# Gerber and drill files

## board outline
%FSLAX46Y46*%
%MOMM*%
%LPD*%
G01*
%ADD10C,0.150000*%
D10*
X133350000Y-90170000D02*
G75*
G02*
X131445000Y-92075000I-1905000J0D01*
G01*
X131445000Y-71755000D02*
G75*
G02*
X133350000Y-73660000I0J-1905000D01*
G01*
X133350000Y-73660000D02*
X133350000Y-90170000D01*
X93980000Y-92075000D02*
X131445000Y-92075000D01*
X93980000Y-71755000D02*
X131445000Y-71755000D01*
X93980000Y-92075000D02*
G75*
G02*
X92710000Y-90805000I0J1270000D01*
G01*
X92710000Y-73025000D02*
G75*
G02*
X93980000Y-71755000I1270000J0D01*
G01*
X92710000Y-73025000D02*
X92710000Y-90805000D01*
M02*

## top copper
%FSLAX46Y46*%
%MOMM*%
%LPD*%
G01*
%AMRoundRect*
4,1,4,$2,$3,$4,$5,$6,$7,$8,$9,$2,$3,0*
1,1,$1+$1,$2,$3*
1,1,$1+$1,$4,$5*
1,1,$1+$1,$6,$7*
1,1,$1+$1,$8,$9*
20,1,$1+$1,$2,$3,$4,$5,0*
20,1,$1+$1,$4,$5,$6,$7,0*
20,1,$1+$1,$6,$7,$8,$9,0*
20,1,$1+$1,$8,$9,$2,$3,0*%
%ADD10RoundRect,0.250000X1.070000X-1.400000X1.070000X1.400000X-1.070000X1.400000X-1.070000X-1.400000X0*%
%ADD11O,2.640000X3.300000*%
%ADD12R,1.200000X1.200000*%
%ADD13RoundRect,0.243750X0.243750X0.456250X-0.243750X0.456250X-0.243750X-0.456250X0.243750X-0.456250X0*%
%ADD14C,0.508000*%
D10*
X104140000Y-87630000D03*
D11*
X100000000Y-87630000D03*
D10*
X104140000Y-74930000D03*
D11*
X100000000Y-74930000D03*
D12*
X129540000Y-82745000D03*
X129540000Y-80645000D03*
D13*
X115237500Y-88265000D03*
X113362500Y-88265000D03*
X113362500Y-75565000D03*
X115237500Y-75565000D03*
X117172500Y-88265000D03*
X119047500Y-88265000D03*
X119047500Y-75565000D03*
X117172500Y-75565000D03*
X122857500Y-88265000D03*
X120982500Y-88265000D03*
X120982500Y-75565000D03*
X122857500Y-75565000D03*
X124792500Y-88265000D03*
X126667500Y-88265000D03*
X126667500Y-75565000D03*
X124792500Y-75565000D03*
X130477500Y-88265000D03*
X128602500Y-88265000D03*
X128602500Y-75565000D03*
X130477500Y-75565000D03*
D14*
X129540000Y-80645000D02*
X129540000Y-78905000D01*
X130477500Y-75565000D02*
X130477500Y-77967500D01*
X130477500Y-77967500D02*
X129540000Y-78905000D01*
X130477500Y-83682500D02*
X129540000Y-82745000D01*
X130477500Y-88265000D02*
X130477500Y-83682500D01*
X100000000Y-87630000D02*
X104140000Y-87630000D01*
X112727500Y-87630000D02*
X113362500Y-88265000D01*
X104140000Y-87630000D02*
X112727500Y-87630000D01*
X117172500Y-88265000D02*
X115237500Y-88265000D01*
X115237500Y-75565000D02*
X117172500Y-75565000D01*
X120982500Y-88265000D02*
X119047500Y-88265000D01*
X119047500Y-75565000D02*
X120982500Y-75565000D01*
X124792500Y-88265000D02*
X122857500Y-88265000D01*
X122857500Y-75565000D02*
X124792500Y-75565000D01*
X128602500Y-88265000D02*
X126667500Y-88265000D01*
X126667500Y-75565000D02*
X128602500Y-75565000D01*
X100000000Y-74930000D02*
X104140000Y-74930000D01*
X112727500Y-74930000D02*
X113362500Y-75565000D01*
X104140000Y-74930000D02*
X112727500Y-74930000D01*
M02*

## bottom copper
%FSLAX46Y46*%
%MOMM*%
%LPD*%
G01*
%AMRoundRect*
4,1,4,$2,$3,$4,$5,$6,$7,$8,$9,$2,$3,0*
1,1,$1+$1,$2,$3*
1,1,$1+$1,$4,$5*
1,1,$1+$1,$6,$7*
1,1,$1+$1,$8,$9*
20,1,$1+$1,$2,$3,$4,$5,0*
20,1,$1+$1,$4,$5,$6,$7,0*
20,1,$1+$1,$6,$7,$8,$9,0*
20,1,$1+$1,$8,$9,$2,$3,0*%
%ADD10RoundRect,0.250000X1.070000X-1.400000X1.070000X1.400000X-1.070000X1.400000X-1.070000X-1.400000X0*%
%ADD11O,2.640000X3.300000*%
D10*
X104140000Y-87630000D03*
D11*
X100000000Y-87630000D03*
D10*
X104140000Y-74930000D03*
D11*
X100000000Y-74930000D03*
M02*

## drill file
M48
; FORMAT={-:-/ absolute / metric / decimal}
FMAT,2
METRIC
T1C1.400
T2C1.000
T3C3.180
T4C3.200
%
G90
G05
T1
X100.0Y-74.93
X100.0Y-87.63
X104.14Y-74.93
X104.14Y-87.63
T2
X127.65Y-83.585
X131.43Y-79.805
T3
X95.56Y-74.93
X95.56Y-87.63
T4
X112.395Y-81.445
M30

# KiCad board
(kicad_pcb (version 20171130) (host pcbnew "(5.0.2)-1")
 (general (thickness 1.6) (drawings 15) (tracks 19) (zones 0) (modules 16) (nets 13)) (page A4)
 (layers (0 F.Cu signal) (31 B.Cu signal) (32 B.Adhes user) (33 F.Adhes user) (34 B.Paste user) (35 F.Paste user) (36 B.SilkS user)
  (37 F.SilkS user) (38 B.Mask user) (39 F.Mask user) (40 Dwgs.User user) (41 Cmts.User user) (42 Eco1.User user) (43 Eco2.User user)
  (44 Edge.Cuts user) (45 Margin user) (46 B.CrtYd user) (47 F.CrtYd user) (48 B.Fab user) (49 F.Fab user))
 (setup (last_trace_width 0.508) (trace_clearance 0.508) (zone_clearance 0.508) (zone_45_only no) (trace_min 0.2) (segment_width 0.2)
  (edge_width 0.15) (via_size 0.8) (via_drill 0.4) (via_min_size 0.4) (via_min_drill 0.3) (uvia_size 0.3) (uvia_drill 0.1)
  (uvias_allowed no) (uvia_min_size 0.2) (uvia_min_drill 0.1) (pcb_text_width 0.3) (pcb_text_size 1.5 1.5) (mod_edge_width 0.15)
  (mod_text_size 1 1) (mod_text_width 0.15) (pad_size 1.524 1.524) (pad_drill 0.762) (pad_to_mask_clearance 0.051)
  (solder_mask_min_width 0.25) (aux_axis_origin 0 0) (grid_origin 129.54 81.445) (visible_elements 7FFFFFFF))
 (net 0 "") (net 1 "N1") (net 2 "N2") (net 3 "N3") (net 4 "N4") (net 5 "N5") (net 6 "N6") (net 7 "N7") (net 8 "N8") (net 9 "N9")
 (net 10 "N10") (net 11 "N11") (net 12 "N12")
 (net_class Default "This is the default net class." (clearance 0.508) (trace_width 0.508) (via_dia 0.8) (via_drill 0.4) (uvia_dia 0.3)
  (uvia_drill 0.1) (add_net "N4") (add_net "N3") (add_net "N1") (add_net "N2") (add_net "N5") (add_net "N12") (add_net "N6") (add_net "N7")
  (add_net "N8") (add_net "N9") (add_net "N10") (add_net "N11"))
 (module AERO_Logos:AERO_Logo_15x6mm (layer F.Cu) (at 101.6 81.445)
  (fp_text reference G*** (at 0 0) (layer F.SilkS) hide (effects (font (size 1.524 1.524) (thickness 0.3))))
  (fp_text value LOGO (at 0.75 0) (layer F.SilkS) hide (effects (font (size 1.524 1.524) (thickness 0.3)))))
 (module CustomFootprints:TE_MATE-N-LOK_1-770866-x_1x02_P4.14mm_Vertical (layer B.Cu) (at 104.14 87.63 90)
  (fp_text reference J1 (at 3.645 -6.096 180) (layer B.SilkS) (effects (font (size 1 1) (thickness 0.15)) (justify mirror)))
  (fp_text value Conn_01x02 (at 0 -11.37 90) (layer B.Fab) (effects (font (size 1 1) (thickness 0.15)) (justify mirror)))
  (pad 1 thru_hole roundrect (at 0 0 90) (size 3.3 2.64) (drill 1.4) (layers *.Cu *.Mask) (roundrect_rratio 0.094697) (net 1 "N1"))
  (pad 2 thru_hole oval (at 0 -4.14 90) (size 3.3 2.64) (drill 1.4) (layers *.Cu *.Mask) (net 1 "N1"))
  (pad "" np_thru_hole circle (at 0 -8.58 90) (size 3.18 3.18) (drill 3.18) (layers *.Cu *.Mask)))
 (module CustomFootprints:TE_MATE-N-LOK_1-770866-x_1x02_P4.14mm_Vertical (layer B.Cu) (at 104.14 74.93 90)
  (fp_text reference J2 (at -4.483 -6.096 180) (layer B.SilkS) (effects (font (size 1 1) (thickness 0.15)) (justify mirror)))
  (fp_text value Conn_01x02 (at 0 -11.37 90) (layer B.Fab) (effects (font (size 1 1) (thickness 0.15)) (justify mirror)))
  (pad 1 thru_hole roundrect (at 0 0 90) (size 3.3 2.64) (drill 1.4) (layers *.Cu *.Mask) (roundrect_rratio 0.094697) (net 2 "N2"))
  (pad 2 thru_hole oval (at 0 -4.14 90) (size 3.3 2.64) (drill 1.4) (layers *.Cu *.Mask) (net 2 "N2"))
  (pad "" np_thru_hole circle (at 0 -8.58 90) (size 3.18 3.18) (drill 3.18) (layers *.Cu *.Mask)))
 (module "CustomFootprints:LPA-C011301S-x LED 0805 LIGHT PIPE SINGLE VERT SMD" (layer F.Cu) (at 129.54 81.695 270)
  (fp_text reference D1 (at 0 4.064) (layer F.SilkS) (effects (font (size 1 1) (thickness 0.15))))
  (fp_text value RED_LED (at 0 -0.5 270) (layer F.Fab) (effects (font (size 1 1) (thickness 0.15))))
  (pad "" np_thru_hole circle (at 1.89 1.89 270) (size 1 1) (drill 1) (layers *.Cu *.Mask))
  (pad "" np_thru_hole circle (at -1.89 -1.89 270) (size 1 1) (drill 1) (layers *.Cu *.Mask))
  (pad 2 smd rect (at 1.05 0 270) (size 1.2 1.2) (layers F.Cu F.Paste F.Mask) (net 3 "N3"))
  (pad 1 smd rect (at -1.05 0 270) (size 1.2 1.2) (layers F.Cu F.Paste F.Mask) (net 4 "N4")))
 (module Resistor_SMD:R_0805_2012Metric (layer F.Cu) (at 114.3 88.265 180)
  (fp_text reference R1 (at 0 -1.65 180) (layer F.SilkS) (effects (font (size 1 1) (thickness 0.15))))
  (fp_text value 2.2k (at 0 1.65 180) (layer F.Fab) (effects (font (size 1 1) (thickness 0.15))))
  (pad 1 smd roundrect (at -0.9375 0 180) (size 0.975 1.4) (layers F.Cu F.Paste F.Mask) (roundrect_rratio 0.25) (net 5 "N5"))
  (pad 2 smd roundrect (at 0.9375 0 180) (size 0.975 1.4) (layers F.Cu F.Paste F.Mask) (roundrect_rratio 0.25) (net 1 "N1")))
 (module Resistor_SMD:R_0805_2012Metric (layer F.Cu) (at 114.3 75.565 180)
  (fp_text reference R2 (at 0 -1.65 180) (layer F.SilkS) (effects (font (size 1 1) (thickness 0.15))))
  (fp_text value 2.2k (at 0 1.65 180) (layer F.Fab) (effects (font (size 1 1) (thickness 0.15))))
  (pad 2 smd roundrect (at 0.9375 0 180) (size 0.975 1.4) (layers F.Cu F.Paste F.Mask) (roundrect_rratio 0.25) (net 2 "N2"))
  (pad 1 smd roundrect (at -0.9375 0 180) (size 0.975 1.4) (layers F.Cu F.Paste F.Mask) (roundrect_rratio 0.25) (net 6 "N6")))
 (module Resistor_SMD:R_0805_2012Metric (layer F.Cu) (at 118.11 88.265 180)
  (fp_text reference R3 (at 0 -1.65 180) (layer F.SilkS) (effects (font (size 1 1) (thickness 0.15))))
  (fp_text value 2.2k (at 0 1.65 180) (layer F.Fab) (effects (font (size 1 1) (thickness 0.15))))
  (pad 2 smd roundrect (at 0.9375 0 180) (size 0.975 1.4) (layers F.Cu F.Paste F.Mask) (roundrect_rratio 0.25) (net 5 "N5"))
  (pad 1 smd roundrect (at -0.9375 0 180) (size 0.975 1.4) (layers F.Cu F.Paste F.Mask) (roundrect_rratio 0.25) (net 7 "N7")))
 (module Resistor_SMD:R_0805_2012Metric (layer F.Cu) (at 118.11 75.565 180)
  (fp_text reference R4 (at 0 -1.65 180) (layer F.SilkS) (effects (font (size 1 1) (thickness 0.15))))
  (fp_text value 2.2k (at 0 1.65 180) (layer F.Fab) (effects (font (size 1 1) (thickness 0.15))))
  (pad 1 smd roundrect (at -0.9375 0 180) (size 0.975 1.4) (layers F.Cu F.Paste F.Mask) (roundrect_rratio 0.25) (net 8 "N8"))
  (pad 2 smd roundrect (at 0.9375 0 180) (size 0.975 1.4) (layers F.Cu F.Paste F.Mask) (roundrect_rratio 0.25) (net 6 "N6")))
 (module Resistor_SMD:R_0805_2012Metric (layer F.Cu) (at 121.92 88.265 180)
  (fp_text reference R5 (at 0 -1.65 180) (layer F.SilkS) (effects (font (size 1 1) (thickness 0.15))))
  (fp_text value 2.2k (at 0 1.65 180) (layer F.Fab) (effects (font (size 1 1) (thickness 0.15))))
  (pad 1 smd roundrect (at -0.9375 0 180) (size 0.975 1.4) (layers F.Cu F.Paste F.Mask) (roundrect_rratio 0.25) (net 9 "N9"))
  (pad 2 smd roundrect (at 0.9375 0 180) (size 0.975 1.4) (layers F.Cu F.Paste F.Mask) (roundrect_rratio 0.25) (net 7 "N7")))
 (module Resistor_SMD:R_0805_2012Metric (layer F.Cu) (at 121.92 75.565 180)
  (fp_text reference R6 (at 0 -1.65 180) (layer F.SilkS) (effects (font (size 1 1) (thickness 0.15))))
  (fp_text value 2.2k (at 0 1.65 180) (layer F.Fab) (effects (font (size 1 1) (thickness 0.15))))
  (pad 2 smd roundrect (at 0.9375 0 180) (size 0.975 1.4) (layers F.Cu F.Paste F.Mask) (roundrect_rratio 0.25) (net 8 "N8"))
  (pad 1 smd roundrect (at -0.9375 0 180) (size 0.975 1.4) (layers F.Cu F.Paste F.Mask) (roundrect_rratio 0.25) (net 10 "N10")))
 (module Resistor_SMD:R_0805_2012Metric (layer F.Cu) (at 125.73 88.265 180)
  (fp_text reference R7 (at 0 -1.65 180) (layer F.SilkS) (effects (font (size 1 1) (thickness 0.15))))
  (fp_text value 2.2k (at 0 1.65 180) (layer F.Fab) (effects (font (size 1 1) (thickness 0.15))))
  (pad 2 smd roundrect (at 0.9375 0 180) (size 0.975 1.4) (layers F.Cu F.Paste F.Mask) (roundrect_rratio 0.25) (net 9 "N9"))
  (pad 1 smd roundrect (at -0.9375 0 180) (size 0.975 1.4) (layers F.Cu F.Paste F.Mask) (roundrect_rratio 0.25) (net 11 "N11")))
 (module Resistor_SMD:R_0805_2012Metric (layer F.Cu) (at 125.73 75.565 180)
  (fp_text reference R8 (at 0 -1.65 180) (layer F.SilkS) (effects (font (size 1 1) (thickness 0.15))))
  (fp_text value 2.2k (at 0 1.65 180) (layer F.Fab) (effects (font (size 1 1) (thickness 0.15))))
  (pad 1 smd roundrect (at -0.9375 0 180) (size 0.975 1.4) (layers F.Cu F.Paste F.Mask) (roundrect_rratio 0.25) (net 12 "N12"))
  (pad 2 smd roundrect (at 0.9375 0 180) (size 0.975 1.4) (layers F.Cu F.Paste F.Mask) (roundrect_rratio 0.25) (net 10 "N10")))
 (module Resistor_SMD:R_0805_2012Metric (layer F.Cu) (at 129.54 88.265 180)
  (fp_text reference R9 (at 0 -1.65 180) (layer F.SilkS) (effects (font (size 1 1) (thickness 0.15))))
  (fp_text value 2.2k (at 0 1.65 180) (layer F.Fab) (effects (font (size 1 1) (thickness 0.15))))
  (pad 1 smd roundrect (at -0.9375 0 180) (size 0.975 1.4) (layers F.Cu F.Paste F.Mask) (roundrect_rratio 0.25) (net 3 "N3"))
  (pad 2 smd roundrect (at 0.9375 0 180) (size 0.975 1.4) (layers F.Cu F.Paste F.Mask) (roundrect_rratio 0.25) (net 11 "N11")))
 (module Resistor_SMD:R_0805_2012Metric (layer F.Cu) (at 129.54 75.565 180)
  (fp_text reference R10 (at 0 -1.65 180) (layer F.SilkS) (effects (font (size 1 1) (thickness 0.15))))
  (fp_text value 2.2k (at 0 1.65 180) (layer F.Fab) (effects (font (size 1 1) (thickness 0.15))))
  (pad 2 smd roundrect (at 0.9375 0 180) (size 0.975 1.4) (layers F.Cu F.Paste F.Mask) (roundrect_rratio 0.25) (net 12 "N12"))
  (pad 1 smd roundrect (at -0.9375 0 180) (size 0.975 1.4) (layers F.Cu F.Paste F.Mask) (roundrect_rratio 0.25) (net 4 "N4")))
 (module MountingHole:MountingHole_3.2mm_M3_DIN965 (layer F.Cu) (at 112.395 81.445)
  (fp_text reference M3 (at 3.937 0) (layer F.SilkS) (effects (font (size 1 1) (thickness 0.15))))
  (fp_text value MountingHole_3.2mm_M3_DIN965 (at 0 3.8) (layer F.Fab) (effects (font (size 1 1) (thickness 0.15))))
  (pad 1 np_thru_hole circle (at 0 0) (size 3.2 3.2) (drill 3.2) (layers *.Cu *.Mask)))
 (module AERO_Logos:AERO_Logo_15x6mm (layer B.Cu) (at 122.936 77.381 180)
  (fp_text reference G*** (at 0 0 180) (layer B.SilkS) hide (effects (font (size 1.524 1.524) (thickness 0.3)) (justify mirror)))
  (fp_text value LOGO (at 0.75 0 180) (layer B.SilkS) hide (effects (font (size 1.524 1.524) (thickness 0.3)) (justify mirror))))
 (gr_arc (start 131.445 90.17) (end 131.445 92.075) (angle -90) (layer Edge.Cuts) (width 0.15))
 (gr_arc (start 131.445 73.66) (end 133.35 73.66) (angle -90) (layer Edge.Cuts) (width 0.15))
 (gr_line (start 133.35 73.66) (end 133.35 90.17) (layer Edge.Cuts) (width 0.15))
 (gr_line (start 93.98 92.075) (end 131.445 92.075) (layer Edge.Cuts) (width 0.15))
 (gr_line (start 93.98 71.755) (end 131.445 71.755) (layer Edge.Cuts) (width 0.15))
 (gr_arc (start 93.98 90.805) (end 92.71 90.805) (angle -90) (layer Edge.Cuts) (width 0.15))
 (gr_arc (start 93.98 73.025) (end 93.98 71.755) (angle -90) (layer Edge.Cuts) (width 0.15))
 (gr_line (start 92.71 73.025) (end 92.71 90.805) (layer Edge.Cuts) (width 0.15))
 (segment (start 129.54 80.645) (end 129.54 78.905) (width 0.508) (layer F.Cu) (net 4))
 (segment (start 130.4775 75.565) (end 130.4775 77.9675) (width 0.508) (layer F.Cu) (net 4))
 (segment (start 130.4775 77.9675) (end 129.54 78.905) (width 0.508) (layer F.Cu) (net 4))
 (segment (start 130.4775 83.6825) (end 129.54 82.745) (width 0.508) (layer F.Cu) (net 3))
 (segment (start 130.4775 88.265) (end 130.4775 83.6825) (width 0.508) (layer F.Cu) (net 3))
 (segment (start 100 87.63) (end 104.14 87.63) (width 0.508) (layer F.Cu) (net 1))
 (segment (start 112.7275 87.63) (end 113.3625 88.265) (width 0.508) (layer F.Cu) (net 1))
 (segment (start 104.14 87.63) (end 112.7275 87.63) (width 0.508) (layer F.Cu) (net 1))
 (segment (start 117.1725 88.265) (end 115.2375 88.265) (width 0.508) (layer F.Cu) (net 5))
 (segment (start 115.2375 75.565) (end 117.1725 75.565) (width 0.508) (layer F.Cu) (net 6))
 (segment (start 120.9825 88.265) (end 119.0475 88.265) (width 0.508) (layer F.Cu) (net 7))
 (segment (start 119.0475 75.565) (end 120.9825 75.565) (width 0.508) (layer F.Cu) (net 8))
 (segment (start 124.7925 88.265) (end 122.8575 88.265) (width 0.508) (layer F.Cu) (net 9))
 (segment (start 122.8575 75.565) (end 124.7925 75.565) (width 0.508) (layer F.Cu) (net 10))
 (segment (start 128.6025 88.265) (end 126.6675 88.265) (width 0.508) (layer F.Cu) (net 11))
 (segment (start 126.6675 75.565) (end 128.6025 75.565) (width 0.508) (layer F.Cu) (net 12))
 (segment (start 100 74.93) (end 104.14 74.93) (width 0.508) (layer F.Cu) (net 2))
 (segment (start 112.7275 74.93) (end 113.3625 75.565) (width 0.508) (layer F.Cu) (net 2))
 (segment (start 104.14 74.93) (end 112.7275 74.93) (width 0.508) (layer F.Cu) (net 2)))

